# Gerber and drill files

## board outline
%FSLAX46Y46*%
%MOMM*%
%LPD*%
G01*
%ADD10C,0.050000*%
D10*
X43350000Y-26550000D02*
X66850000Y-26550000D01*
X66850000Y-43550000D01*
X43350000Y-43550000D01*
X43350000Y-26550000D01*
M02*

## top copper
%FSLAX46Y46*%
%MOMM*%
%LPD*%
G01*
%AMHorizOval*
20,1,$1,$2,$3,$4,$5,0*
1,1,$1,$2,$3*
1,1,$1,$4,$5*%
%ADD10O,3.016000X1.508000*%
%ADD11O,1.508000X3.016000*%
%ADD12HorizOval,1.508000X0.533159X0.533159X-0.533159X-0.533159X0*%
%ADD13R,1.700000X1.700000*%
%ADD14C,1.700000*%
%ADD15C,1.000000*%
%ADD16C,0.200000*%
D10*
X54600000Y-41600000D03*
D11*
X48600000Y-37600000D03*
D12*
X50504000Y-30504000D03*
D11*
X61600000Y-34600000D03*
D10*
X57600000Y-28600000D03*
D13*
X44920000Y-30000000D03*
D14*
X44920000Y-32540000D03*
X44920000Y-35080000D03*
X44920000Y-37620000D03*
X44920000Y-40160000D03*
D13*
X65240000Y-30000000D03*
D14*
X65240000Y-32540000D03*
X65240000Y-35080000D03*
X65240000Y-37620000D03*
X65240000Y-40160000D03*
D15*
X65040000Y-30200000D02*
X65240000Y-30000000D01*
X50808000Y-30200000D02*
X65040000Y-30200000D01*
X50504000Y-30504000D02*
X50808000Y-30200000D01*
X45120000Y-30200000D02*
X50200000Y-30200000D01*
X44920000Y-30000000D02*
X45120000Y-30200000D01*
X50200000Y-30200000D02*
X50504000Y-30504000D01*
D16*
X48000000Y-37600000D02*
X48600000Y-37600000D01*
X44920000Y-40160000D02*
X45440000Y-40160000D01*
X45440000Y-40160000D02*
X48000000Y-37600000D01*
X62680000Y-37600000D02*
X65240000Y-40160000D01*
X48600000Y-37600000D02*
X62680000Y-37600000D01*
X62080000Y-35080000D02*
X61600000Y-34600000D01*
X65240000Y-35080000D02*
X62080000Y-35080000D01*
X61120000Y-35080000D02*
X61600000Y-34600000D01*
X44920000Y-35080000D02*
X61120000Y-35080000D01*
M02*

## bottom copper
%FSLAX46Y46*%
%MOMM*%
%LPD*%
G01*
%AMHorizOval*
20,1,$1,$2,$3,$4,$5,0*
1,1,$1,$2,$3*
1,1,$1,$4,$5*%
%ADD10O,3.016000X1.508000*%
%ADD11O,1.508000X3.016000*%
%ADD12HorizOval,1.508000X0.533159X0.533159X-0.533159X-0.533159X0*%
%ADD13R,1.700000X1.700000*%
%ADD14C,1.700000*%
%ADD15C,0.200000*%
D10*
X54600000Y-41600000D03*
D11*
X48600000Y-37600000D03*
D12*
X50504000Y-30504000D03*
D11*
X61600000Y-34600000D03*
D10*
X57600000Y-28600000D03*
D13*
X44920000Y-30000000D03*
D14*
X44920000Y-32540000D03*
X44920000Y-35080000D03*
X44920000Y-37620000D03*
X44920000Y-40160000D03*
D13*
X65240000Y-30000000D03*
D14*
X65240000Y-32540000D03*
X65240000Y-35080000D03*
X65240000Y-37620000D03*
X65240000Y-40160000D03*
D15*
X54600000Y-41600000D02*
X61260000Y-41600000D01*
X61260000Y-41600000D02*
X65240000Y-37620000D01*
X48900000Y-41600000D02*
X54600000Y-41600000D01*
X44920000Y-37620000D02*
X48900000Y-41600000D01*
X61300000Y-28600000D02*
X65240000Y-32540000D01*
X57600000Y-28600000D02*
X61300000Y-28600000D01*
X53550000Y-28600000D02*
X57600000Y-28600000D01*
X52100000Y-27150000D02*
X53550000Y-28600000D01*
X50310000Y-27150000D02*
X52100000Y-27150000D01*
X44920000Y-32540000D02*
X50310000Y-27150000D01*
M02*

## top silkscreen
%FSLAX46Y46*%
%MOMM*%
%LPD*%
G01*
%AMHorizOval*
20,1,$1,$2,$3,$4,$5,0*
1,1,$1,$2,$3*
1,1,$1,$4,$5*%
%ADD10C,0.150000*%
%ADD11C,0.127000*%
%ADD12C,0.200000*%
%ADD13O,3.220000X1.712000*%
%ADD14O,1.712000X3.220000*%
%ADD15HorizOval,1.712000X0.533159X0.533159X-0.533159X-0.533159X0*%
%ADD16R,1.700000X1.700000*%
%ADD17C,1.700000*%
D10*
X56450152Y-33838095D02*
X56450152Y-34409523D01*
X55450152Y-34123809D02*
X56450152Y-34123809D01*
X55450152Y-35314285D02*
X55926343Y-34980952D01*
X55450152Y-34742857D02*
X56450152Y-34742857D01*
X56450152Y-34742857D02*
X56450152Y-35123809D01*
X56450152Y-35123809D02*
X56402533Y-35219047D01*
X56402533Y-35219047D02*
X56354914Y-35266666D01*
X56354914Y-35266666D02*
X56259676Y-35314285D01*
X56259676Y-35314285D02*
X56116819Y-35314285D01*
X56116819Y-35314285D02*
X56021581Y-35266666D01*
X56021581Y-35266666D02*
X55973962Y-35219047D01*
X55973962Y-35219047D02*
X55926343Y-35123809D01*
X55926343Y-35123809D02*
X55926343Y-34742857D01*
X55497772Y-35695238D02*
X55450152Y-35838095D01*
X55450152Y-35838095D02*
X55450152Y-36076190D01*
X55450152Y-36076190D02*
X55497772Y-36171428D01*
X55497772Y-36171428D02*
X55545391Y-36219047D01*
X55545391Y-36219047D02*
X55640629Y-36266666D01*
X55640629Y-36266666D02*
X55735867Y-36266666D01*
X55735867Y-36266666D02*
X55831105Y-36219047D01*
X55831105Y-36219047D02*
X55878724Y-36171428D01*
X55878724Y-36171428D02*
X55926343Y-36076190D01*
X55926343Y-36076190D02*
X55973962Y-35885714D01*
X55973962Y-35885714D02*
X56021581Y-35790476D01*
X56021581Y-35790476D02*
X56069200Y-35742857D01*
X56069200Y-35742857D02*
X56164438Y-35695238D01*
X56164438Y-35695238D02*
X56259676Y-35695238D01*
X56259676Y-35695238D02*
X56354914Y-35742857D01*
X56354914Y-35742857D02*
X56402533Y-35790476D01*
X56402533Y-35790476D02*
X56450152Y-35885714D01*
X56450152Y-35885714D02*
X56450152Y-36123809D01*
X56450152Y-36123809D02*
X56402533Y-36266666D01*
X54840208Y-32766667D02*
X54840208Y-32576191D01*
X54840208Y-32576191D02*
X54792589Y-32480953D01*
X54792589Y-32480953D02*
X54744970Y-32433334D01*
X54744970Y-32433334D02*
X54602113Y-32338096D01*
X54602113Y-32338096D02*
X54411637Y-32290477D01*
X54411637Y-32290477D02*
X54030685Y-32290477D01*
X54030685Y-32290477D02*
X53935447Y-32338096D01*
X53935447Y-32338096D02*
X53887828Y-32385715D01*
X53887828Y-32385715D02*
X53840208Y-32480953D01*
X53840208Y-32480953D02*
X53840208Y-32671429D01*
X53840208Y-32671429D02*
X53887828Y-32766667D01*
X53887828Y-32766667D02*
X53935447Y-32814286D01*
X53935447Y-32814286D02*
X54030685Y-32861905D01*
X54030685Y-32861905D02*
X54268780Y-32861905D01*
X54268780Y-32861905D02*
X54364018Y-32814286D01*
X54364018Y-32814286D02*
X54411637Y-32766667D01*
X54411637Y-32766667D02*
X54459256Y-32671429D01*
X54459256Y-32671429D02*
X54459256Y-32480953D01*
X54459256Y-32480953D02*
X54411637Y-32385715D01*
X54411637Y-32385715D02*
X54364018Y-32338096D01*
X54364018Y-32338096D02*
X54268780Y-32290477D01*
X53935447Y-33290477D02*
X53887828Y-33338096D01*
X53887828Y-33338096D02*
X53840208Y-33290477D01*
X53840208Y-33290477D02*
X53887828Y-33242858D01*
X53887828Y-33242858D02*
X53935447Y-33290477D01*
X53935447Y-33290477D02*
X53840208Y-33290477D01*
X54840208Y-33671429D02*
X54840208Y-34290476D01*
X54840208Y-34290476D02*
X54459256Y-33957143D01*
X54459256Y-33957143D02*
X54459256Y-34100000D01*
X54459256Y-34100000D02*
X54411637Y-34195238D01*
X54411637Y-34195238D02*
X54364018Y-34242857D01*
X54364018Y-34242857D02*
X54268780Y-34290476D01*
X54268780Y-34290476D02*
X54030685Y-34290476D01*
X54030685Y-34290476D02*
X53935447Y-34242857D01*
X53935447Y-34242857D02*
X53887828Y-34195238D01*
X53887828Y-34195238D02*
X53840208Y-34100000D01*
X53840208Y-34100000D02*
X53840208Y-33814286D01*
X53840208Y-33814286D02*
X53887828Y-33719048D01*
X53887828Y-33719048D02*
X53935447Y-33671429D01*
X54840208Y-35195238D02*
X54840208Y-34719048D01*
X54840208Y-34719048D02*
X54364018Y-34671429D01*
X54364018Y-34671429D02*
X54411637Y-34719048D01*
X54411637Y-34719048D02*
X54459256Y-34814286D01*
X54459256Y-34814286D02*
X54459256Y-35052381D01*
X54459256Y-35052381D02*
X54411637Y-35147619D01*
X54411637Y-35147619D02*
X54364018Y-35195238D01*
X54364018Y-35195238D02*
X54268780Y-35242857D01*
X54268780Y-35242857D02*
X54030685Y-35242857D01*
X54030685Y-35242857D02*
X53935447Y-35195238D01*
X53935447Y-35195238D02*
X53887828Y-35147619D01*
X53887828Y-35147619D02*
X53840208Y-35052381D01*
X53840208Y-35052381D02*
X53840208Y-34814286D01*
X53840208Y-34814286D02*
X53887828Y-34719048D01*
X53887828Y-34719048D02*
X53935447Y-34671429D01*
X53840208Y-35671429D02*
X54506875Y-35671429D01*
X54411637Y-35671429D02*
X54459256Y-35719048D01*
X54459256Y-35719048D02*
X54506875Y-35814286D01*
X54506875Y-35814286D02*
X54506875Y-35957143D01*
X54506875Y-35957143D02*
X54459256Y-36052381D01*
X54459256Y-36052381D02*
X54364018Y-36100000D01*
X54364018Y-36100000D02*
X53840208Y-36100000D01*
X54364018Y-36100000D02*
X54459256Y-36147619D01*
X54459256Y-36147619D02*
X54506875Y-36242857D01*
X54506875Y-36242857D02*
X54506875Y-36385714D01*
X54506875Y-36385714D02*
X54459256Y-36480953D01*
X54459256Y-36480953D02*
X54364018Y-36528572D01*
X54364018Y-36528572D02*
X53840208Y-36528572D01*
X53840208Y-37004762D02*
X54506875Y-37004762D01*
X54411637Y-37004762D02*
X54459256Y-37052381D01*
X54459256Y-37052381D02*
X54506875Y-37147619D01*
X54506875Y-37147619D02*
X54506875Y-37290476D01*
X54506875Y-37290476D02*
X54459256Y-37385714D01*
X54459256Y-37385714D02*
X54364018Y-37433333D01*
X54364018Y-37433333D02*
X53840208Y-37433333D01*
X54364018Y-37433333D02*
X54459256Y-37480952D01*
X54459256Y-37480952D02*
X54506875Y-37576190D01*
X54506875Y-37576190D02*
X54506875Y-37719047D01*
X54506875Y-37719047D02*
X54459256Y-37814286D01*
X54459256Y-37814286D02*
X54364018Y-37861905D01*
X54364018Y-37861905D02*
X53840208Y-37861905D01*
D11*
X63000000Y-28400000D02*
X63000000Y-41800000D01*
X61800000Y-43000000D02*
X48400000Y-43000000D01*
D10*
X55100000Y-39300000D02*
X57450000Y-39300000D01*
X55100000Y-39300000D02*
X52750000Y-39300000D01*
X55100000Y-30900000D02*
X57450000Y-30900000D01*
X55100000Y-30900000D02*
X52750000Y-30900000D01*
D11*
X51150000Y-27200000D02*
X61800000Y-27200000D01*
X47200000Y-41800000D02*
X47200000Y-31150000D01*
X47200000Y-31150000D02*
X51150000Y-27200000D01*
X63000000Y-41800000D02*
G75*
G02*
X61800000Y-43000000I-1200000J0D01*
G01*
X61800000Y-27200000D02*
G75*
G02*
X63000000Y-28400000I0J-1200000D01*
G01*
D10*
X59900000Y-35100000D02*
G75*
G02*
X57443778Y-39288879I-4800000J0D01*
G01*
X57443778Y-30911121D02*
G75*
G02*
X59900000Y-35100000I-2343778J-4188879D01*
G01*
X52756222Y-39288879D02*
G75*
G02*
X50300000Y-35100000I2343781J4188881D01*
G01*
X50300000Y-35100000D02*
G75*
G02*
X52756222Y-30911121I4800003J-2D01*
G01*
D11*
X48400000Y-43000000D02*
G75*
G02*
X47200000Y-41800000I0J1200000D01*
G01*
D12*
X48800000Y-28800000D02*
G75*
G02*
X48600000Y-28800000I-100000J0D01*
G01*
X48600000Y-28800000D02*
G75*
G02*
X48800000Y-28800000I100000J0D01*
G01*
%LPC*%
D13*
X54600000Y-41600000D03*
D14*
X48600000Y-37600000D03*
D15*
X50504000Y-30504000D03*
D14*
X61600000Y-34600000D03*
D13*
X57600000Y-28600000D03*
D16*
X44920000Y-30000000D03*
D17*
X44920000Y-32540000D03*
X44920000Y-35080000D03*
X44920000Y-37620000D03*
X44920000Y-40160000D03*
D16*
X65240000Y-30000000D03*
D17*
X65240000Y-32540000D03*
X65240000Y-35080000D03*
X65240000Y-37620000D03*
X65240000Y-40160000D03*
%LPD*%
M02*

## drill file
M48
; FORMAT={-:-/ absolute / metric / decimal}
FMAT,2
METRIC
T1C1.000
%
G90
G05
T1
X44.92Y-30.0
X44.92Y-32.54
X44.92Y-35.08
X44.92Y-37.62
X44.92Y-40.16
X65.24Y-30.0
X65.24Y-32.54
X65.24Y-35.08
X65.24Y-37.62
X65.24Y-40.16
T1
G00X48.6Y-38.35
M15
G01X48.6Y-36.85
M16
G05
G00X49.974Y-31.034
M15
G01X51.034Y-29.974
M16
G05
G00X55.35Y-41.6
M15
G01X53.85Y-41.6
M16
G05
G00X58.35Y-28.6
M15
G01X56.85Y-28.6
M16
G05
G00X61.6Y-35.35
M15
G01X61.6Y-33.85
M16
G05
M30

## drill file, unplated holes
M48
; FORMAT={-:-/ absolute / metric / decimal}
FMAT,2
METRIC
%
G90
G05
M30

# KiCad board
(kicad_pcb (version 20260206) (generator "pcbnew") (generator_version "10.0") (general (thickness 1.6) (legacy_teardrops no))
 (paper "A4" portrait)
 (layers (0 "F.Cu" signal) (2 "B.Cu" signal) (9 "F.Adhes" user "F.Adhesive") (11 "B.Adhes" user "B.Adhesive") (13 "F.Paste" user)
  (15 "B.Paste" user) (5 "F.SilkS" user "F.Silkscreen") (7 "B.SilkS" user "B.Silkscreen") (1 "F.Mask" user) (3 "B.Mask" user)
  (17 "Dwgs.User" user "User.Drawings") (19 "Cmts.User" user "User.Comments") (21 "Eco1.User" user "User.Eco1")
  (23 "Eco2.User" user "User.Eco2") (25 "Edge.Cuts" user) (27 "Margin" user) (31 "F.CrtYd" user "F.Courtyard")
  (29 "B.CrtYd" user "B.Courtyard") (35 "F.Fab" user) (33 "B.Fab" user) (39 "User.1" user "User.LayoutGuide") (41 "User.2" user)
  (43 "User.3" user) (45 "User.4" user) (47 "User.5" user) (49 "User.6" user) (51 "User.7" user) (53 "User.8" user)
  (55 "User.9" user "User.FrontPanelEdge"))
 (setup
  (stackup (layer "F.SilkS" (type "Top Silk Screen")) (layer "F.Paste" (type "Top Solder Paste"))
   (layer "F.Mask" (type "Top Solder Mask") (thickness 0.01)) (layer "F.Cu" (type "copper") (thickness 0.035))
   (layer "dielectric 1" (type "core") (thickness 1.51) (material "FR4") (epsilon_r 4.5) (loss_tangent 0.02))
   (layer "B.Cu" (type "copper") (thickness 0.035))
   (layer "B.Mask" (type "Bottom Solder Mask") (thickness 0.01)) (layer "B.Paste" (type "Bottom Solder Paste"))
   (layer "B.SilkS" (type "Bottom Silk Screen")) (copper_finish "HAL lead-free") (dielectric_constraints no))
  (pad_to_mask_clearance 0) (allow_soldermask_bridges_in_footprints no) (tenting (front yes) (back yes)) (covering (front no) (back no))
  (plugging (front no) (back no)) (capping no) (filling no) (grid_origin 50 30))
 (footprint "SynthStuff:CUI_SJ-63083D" (layer "F.Cu") (at 55.1 35.1 180)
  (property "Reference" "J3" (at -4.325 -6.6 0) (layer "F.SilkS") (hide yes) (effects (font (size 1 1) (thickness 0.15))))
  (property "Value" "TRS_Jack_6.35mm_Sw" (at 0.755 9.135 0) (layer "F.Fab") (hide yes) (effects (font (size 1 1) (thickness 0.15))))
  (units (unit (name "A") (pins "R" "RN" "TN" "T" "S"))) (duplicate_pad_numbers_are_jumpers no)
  (fp_line (start 7.9 3.95) (end 3.95 7.9) (stroke (width 0.127) (type solid)) (layer "F.SilkS"))
  (fp_line (start 7.9 -6.7) (end 7.9 3.95) (stroke (width 0.127) (type solid)) (layer "F.SilkS"))
  (fp_line (start 3.95 7.9) (end -6.7 7.9) (stroke (width 0.127) (type solid)) (layer "F.SilkS"))
  (fp_line (start 0 4.2) (end 2.35 4.2) (stroke (width 0.15) (type default)) (layer "F.SilkS"))
  (fp_line (start 0 4.2) (end -2.35 4.2) (stroke (width 0.15) (type default)) (layer "F.SilkS"))
  (fp_line (start 0 -4.2) (end 2.35 -4.2) (stroke (width 0.15) (type default)) (layer "F.SilkS"))
  (fp_line (start 0 -4.2) (end -2.35 -4.2) (stroke (width 0.15) (type default)) (layer "F.SilkS"))
  (fp_line (start -6.7 -7.9) (end 6.7 -7.9) (stroke (width 0.127) (type solid)) (layer "F.SilkS"))
  (fp_line (start -7.9 6.7) (end -7.9 -6.7) (stroke (width 0.127) (type solid)) (layer "F.SilkS"))
  (fp_arc (start 6.7 -7.9) (mid 7.548528 -7.548528) (end 7.9 -6.7) (stroke (width 0.127) (type solid)) (layer "F.SilkS"))
  (fp_arc (start 4.8 0) (mid 4.14066 2.427948) (end 2.343778 4.188879) (stroke (width 0.15) (type default)) (layer "F.SilkS"))
  (fp_arc (start 2.343778 -4.188879) (mid 4.14066 -2.427948) (end 4.8 0) (stroke (width 0.15) (type default)) (layer "F.SilkS"))
  (fp_arc (start -2.343778 4.188879) (mid -4.14066 2.427948) (end -4.8 0) (stroke (width 0.15) (type default)) (layer "F.SilkS"))
  (fp_arc (start -4.8 0) (mid -4.14066 -2.427948) (end -2.343778 -4.188879) (stroke (width 0.15) (type default)) (layer "F.SilkS"))
  (fp_arc (start -6.7 7.9) (mid -7.548528 7.548528) (end -7.9 6.7) (stroke (width 0.127) (type solid)) (layer "F.SilkS"))
  (fp_arc (start -7.9 -6.7) (mid -7.548528 -7.548528) (end -6.7 -7.9) (stroke (width 0.127) (type solid)) (layer "F.SilkS"))
  (fp_circle (center 6.4 6.3) (end 6.5 6.3) (stroke (width 0.2) (type solid)) (fill no) (layer "F.SilkS"))
  (pad "R" thru_hole oval (at 0.5 -6.5 180) (size 3.016 1.508) (drill oval 2.5 1) (layers "*.Cu" "*.Mask") (remove_unused_layers no)
   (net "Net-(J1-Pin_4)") (solder_mask_margin 0.102))
  (pad "RN" thru_hole oval (at 6.5 -2.5 180) (size 1.508 3.016) (drill oval 1 2.5) (layers "*.Cu" "*.Mask") (remove_unused_layers no)
   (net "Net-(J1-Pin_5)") (solder_mask_margin 0.102))
  (pad "S" thru_hole oval (at 4.596 4.596 45) (size 3.016 1.508) (drill oval 2.49999 1) (layers "*.Cu" "*.Mask") (remove_unused_layers no)
   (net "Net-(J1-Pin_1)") (solder_mask_margin 0.102))
  (pad "T" thru_hole oval (at -6.5 0.5 180) (size 1.508 3.016) (drill oval 1 2.5) (layers "*.Cu" "*.Mask") (remove_unused_layers no)
   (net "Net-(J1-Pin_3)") (solder_mask_margin 0.102))
  (pad "TN" thru_hole oval (at -2.5 6.5 180) (size 3.016 1.508) (drill oval 2.5 1) (layers "*.Cu" "*.Mask") (remove_unused_layers no)
   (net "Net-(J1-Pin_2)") (solder_mask_margin 0.102)))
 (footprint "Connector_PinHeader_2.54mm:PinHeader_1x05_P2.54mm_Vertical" (layer "B.Cu") (at 44.92 30 180)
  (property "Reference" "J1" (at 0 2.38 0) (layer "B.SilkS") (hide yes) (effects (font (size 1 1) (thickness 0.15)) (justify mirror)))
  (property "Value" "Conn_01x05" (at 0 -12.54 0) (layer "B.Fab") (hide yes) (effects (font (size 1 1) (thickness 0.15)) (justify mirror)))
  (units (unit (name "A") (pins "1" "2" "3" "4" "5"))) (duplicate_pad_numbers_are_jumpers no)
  (pad "1" thru_hole rect (at 0 0 180) (size 1.7 1.7) (drill 1) (layers "*.Cu" "*.Mask") (remove_unused_layers no) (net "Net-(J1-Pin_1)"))
  (pad "2" thru_hole circle (at 0 -2.54 180) (size 1.7 1.7) (drill 1) (layers "*.Cu" "*.Mask") (remove_unused_layers no)
   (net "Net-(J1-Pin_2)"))
  (pad "3" thru_hole circle (at 0 -5.08 180) (size 1.7 1.7) (drill 1) (layers "*.Cu" "*.Mask") (remove_unused_layers no)
   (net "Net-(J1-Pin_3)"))
  (pad "4" thru_hole circle (at 0 -7.62 180) (size 1.7 1.7) (drill 1) (layers "*.Cu" "*.Mask") (remove_unused_layers no)
   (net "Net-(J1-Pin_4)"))
  (pad "5" thru_hole circle (at 0 -10.16 180) (size 1.7 1.7) (drill 1) (layers "*.Cu" "*.Mask") (remove_unused_layers no)
   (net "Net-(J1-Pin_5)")))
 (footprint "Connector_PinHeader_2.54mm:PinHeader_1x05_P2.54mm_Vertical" (layer "B.Cu") (at 65.24 30 180)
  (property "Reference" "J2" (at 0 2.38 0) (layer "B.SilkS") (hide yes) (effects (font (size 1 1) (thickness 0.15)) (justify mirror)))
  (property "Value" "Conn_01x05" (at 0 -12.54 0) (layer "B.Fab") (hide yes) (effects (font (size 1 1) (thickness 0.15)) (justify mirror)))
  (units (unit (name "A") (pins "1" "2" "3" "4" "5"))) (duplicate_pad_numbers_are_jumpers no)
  (pad "1" thru_hole rect (at 0 0 180) (size 1.7 1.7) (drill 1) (layers "*.Cu" "*.Mask") (remove_unused_layers no) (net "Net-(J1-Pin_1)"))
  (pad "2" thru_hole circle (at 0 -2.54 180) (size 1.7 1.7) (drill 1) (layers "*.Cu" "*.Mask") (remove_unused_layers no)
   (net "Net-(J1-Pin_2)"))
  (pad "3" thru_hole circle (at 0 -5.08 180) (size 1.7 1.7) (drill 1) (layers "*.Cu" "*.Mask") (remove_unused_layers no)
   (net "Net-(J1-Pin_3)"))
  (pad "4" thru_hole circle (at 0 -7.62 180) (size 1.7 1.7) (drill 1) (layers "*.Cu" "*.Mask") (remove_unused_layers no)
   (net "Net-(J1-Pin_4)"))
  (pad "5" thru_hole circle (at 0 -10.16 180) (size 1.7 1.7) (drill 1) (layers "*.Cu" "*.Mask") (remove_unused_layers no)
   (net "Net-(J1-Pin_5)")))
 (gr_rect (start 43.35 26.55) (end 66.85 43.55) (stroke (width 0.05) (type solid)) (fill no) (layer "Edge.Cuts"))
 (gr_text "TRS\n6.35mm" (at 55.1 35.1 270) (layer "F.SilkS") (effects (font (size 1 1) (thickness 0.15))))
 (segment (start 50.504 30.504) (end 50.808 30.2) (width 1) (layer "F.Cu") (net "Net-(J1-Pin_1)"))
 (segment (start 65.04 30.2) (end 65.24 30) (width 1) (layer "F.Cu") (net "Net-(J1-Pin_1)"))
 (segment (start 50.808 30.2) (end 65.04 30.2) (width 1) (layer "F.Cu") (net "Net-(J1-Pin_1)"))
 (segment (start 50.2 30.2) (end 50.504 30.504) (width 1) (layer "F.Cu") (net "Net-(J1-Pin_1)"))
 (segment (start 44.92 30) (end 45.12 30.2) (width 1) (layer "F.Cu") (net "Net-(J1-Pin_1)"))
 (segment (start 45.12 30.2) (end 50.2 30.2) (width 1) (layer "F.Cu") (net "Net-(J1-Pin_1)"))
 (segment (start 44.92 32.54) (end 50.31 27.15) (width 0.2) (layer "B.Cu") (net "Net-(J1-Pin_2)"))
 (segment (start 50.31 27.15) (end 52.1 27.15) (width 0.2) (layer "B.Cu") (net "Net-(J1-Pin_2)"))
 (segment (start 61.3 28.6) (end 65.24 32.54) (width 0.2) (layer "B.Cu") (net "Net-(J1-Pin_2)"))
 (segment (start 57.6 28.6) (end 61.3 28.6) (width 0.2) (layer "B.Cu") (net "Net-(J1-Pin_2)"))
 (segment (start 52.1 27.15) (end 53.55 28.6) (width 0.2) (layer "B.Cu") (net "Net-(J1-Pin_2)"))
 (segment (start 53.55 28.6) (end 57.6 28.6) (width 0.2) (layer "B.Cu") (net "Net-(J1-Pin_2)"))
 (segment (start 62.08 35.08) (end 61.6 34.6) (width 0.2) (layer "F.Cu") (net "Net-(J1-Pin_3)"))
 (segment (start 44.92 35.08) (end 61.12 35.08) (width 0.2) (layer "F.Cu") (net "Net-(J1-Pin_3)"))
 (segment (start 65.24 35.08) (end 62.08 35.08) (width 0.2) (layer "F.Cu") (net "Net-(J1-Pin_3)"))
 (segment (start 61.12 35.08) (end 61.6 34.6) (width 0.2) (layer "F.Cu") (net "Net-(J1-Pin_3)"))
 (segment (start 48.9 41.6) (end 54.6 41.6) (width 0.2) (layer "B.Cu") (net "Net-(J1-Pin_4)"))
 (segment (start 61.26 41.6) (end 65.24 37.62) (width 0.2) (layer "B.Cu") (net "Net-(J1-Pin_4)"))
 (segment (start 44.92 37.62) (end 48.9 41.6) (width 0.2) (layer "B.Cu") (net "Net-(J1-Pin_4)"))
 (segment (start 54.6 41.6) (end 61.26 41.6) (width 0.2) (layer "B.Cu") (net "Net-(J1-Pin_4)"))
 (segment (start 48.6 37.6) (end 62.68 37.6) (width 0.2) (layer "F.Cu") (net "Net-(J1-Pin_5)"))
 (segment (start 62.68 37.6) (end 65.24 40.16) (width 0.2) (layer "F.Cu") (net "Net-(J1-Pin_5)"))
 (segment (start 44.92 40.16) (end 45.44 40.16) (width 0.2) (layer "F.Cu") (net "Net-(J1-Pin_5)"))
 (segment (start 45.44 40.16) (end 48 37.6) (width 0.2) (layer "F.Cu") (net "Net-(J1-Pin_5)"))
 (segment (start 48 37.6) (end 48.6 37.6) (width 0.2) (layer "F.Cu") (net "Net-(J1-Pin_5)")))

